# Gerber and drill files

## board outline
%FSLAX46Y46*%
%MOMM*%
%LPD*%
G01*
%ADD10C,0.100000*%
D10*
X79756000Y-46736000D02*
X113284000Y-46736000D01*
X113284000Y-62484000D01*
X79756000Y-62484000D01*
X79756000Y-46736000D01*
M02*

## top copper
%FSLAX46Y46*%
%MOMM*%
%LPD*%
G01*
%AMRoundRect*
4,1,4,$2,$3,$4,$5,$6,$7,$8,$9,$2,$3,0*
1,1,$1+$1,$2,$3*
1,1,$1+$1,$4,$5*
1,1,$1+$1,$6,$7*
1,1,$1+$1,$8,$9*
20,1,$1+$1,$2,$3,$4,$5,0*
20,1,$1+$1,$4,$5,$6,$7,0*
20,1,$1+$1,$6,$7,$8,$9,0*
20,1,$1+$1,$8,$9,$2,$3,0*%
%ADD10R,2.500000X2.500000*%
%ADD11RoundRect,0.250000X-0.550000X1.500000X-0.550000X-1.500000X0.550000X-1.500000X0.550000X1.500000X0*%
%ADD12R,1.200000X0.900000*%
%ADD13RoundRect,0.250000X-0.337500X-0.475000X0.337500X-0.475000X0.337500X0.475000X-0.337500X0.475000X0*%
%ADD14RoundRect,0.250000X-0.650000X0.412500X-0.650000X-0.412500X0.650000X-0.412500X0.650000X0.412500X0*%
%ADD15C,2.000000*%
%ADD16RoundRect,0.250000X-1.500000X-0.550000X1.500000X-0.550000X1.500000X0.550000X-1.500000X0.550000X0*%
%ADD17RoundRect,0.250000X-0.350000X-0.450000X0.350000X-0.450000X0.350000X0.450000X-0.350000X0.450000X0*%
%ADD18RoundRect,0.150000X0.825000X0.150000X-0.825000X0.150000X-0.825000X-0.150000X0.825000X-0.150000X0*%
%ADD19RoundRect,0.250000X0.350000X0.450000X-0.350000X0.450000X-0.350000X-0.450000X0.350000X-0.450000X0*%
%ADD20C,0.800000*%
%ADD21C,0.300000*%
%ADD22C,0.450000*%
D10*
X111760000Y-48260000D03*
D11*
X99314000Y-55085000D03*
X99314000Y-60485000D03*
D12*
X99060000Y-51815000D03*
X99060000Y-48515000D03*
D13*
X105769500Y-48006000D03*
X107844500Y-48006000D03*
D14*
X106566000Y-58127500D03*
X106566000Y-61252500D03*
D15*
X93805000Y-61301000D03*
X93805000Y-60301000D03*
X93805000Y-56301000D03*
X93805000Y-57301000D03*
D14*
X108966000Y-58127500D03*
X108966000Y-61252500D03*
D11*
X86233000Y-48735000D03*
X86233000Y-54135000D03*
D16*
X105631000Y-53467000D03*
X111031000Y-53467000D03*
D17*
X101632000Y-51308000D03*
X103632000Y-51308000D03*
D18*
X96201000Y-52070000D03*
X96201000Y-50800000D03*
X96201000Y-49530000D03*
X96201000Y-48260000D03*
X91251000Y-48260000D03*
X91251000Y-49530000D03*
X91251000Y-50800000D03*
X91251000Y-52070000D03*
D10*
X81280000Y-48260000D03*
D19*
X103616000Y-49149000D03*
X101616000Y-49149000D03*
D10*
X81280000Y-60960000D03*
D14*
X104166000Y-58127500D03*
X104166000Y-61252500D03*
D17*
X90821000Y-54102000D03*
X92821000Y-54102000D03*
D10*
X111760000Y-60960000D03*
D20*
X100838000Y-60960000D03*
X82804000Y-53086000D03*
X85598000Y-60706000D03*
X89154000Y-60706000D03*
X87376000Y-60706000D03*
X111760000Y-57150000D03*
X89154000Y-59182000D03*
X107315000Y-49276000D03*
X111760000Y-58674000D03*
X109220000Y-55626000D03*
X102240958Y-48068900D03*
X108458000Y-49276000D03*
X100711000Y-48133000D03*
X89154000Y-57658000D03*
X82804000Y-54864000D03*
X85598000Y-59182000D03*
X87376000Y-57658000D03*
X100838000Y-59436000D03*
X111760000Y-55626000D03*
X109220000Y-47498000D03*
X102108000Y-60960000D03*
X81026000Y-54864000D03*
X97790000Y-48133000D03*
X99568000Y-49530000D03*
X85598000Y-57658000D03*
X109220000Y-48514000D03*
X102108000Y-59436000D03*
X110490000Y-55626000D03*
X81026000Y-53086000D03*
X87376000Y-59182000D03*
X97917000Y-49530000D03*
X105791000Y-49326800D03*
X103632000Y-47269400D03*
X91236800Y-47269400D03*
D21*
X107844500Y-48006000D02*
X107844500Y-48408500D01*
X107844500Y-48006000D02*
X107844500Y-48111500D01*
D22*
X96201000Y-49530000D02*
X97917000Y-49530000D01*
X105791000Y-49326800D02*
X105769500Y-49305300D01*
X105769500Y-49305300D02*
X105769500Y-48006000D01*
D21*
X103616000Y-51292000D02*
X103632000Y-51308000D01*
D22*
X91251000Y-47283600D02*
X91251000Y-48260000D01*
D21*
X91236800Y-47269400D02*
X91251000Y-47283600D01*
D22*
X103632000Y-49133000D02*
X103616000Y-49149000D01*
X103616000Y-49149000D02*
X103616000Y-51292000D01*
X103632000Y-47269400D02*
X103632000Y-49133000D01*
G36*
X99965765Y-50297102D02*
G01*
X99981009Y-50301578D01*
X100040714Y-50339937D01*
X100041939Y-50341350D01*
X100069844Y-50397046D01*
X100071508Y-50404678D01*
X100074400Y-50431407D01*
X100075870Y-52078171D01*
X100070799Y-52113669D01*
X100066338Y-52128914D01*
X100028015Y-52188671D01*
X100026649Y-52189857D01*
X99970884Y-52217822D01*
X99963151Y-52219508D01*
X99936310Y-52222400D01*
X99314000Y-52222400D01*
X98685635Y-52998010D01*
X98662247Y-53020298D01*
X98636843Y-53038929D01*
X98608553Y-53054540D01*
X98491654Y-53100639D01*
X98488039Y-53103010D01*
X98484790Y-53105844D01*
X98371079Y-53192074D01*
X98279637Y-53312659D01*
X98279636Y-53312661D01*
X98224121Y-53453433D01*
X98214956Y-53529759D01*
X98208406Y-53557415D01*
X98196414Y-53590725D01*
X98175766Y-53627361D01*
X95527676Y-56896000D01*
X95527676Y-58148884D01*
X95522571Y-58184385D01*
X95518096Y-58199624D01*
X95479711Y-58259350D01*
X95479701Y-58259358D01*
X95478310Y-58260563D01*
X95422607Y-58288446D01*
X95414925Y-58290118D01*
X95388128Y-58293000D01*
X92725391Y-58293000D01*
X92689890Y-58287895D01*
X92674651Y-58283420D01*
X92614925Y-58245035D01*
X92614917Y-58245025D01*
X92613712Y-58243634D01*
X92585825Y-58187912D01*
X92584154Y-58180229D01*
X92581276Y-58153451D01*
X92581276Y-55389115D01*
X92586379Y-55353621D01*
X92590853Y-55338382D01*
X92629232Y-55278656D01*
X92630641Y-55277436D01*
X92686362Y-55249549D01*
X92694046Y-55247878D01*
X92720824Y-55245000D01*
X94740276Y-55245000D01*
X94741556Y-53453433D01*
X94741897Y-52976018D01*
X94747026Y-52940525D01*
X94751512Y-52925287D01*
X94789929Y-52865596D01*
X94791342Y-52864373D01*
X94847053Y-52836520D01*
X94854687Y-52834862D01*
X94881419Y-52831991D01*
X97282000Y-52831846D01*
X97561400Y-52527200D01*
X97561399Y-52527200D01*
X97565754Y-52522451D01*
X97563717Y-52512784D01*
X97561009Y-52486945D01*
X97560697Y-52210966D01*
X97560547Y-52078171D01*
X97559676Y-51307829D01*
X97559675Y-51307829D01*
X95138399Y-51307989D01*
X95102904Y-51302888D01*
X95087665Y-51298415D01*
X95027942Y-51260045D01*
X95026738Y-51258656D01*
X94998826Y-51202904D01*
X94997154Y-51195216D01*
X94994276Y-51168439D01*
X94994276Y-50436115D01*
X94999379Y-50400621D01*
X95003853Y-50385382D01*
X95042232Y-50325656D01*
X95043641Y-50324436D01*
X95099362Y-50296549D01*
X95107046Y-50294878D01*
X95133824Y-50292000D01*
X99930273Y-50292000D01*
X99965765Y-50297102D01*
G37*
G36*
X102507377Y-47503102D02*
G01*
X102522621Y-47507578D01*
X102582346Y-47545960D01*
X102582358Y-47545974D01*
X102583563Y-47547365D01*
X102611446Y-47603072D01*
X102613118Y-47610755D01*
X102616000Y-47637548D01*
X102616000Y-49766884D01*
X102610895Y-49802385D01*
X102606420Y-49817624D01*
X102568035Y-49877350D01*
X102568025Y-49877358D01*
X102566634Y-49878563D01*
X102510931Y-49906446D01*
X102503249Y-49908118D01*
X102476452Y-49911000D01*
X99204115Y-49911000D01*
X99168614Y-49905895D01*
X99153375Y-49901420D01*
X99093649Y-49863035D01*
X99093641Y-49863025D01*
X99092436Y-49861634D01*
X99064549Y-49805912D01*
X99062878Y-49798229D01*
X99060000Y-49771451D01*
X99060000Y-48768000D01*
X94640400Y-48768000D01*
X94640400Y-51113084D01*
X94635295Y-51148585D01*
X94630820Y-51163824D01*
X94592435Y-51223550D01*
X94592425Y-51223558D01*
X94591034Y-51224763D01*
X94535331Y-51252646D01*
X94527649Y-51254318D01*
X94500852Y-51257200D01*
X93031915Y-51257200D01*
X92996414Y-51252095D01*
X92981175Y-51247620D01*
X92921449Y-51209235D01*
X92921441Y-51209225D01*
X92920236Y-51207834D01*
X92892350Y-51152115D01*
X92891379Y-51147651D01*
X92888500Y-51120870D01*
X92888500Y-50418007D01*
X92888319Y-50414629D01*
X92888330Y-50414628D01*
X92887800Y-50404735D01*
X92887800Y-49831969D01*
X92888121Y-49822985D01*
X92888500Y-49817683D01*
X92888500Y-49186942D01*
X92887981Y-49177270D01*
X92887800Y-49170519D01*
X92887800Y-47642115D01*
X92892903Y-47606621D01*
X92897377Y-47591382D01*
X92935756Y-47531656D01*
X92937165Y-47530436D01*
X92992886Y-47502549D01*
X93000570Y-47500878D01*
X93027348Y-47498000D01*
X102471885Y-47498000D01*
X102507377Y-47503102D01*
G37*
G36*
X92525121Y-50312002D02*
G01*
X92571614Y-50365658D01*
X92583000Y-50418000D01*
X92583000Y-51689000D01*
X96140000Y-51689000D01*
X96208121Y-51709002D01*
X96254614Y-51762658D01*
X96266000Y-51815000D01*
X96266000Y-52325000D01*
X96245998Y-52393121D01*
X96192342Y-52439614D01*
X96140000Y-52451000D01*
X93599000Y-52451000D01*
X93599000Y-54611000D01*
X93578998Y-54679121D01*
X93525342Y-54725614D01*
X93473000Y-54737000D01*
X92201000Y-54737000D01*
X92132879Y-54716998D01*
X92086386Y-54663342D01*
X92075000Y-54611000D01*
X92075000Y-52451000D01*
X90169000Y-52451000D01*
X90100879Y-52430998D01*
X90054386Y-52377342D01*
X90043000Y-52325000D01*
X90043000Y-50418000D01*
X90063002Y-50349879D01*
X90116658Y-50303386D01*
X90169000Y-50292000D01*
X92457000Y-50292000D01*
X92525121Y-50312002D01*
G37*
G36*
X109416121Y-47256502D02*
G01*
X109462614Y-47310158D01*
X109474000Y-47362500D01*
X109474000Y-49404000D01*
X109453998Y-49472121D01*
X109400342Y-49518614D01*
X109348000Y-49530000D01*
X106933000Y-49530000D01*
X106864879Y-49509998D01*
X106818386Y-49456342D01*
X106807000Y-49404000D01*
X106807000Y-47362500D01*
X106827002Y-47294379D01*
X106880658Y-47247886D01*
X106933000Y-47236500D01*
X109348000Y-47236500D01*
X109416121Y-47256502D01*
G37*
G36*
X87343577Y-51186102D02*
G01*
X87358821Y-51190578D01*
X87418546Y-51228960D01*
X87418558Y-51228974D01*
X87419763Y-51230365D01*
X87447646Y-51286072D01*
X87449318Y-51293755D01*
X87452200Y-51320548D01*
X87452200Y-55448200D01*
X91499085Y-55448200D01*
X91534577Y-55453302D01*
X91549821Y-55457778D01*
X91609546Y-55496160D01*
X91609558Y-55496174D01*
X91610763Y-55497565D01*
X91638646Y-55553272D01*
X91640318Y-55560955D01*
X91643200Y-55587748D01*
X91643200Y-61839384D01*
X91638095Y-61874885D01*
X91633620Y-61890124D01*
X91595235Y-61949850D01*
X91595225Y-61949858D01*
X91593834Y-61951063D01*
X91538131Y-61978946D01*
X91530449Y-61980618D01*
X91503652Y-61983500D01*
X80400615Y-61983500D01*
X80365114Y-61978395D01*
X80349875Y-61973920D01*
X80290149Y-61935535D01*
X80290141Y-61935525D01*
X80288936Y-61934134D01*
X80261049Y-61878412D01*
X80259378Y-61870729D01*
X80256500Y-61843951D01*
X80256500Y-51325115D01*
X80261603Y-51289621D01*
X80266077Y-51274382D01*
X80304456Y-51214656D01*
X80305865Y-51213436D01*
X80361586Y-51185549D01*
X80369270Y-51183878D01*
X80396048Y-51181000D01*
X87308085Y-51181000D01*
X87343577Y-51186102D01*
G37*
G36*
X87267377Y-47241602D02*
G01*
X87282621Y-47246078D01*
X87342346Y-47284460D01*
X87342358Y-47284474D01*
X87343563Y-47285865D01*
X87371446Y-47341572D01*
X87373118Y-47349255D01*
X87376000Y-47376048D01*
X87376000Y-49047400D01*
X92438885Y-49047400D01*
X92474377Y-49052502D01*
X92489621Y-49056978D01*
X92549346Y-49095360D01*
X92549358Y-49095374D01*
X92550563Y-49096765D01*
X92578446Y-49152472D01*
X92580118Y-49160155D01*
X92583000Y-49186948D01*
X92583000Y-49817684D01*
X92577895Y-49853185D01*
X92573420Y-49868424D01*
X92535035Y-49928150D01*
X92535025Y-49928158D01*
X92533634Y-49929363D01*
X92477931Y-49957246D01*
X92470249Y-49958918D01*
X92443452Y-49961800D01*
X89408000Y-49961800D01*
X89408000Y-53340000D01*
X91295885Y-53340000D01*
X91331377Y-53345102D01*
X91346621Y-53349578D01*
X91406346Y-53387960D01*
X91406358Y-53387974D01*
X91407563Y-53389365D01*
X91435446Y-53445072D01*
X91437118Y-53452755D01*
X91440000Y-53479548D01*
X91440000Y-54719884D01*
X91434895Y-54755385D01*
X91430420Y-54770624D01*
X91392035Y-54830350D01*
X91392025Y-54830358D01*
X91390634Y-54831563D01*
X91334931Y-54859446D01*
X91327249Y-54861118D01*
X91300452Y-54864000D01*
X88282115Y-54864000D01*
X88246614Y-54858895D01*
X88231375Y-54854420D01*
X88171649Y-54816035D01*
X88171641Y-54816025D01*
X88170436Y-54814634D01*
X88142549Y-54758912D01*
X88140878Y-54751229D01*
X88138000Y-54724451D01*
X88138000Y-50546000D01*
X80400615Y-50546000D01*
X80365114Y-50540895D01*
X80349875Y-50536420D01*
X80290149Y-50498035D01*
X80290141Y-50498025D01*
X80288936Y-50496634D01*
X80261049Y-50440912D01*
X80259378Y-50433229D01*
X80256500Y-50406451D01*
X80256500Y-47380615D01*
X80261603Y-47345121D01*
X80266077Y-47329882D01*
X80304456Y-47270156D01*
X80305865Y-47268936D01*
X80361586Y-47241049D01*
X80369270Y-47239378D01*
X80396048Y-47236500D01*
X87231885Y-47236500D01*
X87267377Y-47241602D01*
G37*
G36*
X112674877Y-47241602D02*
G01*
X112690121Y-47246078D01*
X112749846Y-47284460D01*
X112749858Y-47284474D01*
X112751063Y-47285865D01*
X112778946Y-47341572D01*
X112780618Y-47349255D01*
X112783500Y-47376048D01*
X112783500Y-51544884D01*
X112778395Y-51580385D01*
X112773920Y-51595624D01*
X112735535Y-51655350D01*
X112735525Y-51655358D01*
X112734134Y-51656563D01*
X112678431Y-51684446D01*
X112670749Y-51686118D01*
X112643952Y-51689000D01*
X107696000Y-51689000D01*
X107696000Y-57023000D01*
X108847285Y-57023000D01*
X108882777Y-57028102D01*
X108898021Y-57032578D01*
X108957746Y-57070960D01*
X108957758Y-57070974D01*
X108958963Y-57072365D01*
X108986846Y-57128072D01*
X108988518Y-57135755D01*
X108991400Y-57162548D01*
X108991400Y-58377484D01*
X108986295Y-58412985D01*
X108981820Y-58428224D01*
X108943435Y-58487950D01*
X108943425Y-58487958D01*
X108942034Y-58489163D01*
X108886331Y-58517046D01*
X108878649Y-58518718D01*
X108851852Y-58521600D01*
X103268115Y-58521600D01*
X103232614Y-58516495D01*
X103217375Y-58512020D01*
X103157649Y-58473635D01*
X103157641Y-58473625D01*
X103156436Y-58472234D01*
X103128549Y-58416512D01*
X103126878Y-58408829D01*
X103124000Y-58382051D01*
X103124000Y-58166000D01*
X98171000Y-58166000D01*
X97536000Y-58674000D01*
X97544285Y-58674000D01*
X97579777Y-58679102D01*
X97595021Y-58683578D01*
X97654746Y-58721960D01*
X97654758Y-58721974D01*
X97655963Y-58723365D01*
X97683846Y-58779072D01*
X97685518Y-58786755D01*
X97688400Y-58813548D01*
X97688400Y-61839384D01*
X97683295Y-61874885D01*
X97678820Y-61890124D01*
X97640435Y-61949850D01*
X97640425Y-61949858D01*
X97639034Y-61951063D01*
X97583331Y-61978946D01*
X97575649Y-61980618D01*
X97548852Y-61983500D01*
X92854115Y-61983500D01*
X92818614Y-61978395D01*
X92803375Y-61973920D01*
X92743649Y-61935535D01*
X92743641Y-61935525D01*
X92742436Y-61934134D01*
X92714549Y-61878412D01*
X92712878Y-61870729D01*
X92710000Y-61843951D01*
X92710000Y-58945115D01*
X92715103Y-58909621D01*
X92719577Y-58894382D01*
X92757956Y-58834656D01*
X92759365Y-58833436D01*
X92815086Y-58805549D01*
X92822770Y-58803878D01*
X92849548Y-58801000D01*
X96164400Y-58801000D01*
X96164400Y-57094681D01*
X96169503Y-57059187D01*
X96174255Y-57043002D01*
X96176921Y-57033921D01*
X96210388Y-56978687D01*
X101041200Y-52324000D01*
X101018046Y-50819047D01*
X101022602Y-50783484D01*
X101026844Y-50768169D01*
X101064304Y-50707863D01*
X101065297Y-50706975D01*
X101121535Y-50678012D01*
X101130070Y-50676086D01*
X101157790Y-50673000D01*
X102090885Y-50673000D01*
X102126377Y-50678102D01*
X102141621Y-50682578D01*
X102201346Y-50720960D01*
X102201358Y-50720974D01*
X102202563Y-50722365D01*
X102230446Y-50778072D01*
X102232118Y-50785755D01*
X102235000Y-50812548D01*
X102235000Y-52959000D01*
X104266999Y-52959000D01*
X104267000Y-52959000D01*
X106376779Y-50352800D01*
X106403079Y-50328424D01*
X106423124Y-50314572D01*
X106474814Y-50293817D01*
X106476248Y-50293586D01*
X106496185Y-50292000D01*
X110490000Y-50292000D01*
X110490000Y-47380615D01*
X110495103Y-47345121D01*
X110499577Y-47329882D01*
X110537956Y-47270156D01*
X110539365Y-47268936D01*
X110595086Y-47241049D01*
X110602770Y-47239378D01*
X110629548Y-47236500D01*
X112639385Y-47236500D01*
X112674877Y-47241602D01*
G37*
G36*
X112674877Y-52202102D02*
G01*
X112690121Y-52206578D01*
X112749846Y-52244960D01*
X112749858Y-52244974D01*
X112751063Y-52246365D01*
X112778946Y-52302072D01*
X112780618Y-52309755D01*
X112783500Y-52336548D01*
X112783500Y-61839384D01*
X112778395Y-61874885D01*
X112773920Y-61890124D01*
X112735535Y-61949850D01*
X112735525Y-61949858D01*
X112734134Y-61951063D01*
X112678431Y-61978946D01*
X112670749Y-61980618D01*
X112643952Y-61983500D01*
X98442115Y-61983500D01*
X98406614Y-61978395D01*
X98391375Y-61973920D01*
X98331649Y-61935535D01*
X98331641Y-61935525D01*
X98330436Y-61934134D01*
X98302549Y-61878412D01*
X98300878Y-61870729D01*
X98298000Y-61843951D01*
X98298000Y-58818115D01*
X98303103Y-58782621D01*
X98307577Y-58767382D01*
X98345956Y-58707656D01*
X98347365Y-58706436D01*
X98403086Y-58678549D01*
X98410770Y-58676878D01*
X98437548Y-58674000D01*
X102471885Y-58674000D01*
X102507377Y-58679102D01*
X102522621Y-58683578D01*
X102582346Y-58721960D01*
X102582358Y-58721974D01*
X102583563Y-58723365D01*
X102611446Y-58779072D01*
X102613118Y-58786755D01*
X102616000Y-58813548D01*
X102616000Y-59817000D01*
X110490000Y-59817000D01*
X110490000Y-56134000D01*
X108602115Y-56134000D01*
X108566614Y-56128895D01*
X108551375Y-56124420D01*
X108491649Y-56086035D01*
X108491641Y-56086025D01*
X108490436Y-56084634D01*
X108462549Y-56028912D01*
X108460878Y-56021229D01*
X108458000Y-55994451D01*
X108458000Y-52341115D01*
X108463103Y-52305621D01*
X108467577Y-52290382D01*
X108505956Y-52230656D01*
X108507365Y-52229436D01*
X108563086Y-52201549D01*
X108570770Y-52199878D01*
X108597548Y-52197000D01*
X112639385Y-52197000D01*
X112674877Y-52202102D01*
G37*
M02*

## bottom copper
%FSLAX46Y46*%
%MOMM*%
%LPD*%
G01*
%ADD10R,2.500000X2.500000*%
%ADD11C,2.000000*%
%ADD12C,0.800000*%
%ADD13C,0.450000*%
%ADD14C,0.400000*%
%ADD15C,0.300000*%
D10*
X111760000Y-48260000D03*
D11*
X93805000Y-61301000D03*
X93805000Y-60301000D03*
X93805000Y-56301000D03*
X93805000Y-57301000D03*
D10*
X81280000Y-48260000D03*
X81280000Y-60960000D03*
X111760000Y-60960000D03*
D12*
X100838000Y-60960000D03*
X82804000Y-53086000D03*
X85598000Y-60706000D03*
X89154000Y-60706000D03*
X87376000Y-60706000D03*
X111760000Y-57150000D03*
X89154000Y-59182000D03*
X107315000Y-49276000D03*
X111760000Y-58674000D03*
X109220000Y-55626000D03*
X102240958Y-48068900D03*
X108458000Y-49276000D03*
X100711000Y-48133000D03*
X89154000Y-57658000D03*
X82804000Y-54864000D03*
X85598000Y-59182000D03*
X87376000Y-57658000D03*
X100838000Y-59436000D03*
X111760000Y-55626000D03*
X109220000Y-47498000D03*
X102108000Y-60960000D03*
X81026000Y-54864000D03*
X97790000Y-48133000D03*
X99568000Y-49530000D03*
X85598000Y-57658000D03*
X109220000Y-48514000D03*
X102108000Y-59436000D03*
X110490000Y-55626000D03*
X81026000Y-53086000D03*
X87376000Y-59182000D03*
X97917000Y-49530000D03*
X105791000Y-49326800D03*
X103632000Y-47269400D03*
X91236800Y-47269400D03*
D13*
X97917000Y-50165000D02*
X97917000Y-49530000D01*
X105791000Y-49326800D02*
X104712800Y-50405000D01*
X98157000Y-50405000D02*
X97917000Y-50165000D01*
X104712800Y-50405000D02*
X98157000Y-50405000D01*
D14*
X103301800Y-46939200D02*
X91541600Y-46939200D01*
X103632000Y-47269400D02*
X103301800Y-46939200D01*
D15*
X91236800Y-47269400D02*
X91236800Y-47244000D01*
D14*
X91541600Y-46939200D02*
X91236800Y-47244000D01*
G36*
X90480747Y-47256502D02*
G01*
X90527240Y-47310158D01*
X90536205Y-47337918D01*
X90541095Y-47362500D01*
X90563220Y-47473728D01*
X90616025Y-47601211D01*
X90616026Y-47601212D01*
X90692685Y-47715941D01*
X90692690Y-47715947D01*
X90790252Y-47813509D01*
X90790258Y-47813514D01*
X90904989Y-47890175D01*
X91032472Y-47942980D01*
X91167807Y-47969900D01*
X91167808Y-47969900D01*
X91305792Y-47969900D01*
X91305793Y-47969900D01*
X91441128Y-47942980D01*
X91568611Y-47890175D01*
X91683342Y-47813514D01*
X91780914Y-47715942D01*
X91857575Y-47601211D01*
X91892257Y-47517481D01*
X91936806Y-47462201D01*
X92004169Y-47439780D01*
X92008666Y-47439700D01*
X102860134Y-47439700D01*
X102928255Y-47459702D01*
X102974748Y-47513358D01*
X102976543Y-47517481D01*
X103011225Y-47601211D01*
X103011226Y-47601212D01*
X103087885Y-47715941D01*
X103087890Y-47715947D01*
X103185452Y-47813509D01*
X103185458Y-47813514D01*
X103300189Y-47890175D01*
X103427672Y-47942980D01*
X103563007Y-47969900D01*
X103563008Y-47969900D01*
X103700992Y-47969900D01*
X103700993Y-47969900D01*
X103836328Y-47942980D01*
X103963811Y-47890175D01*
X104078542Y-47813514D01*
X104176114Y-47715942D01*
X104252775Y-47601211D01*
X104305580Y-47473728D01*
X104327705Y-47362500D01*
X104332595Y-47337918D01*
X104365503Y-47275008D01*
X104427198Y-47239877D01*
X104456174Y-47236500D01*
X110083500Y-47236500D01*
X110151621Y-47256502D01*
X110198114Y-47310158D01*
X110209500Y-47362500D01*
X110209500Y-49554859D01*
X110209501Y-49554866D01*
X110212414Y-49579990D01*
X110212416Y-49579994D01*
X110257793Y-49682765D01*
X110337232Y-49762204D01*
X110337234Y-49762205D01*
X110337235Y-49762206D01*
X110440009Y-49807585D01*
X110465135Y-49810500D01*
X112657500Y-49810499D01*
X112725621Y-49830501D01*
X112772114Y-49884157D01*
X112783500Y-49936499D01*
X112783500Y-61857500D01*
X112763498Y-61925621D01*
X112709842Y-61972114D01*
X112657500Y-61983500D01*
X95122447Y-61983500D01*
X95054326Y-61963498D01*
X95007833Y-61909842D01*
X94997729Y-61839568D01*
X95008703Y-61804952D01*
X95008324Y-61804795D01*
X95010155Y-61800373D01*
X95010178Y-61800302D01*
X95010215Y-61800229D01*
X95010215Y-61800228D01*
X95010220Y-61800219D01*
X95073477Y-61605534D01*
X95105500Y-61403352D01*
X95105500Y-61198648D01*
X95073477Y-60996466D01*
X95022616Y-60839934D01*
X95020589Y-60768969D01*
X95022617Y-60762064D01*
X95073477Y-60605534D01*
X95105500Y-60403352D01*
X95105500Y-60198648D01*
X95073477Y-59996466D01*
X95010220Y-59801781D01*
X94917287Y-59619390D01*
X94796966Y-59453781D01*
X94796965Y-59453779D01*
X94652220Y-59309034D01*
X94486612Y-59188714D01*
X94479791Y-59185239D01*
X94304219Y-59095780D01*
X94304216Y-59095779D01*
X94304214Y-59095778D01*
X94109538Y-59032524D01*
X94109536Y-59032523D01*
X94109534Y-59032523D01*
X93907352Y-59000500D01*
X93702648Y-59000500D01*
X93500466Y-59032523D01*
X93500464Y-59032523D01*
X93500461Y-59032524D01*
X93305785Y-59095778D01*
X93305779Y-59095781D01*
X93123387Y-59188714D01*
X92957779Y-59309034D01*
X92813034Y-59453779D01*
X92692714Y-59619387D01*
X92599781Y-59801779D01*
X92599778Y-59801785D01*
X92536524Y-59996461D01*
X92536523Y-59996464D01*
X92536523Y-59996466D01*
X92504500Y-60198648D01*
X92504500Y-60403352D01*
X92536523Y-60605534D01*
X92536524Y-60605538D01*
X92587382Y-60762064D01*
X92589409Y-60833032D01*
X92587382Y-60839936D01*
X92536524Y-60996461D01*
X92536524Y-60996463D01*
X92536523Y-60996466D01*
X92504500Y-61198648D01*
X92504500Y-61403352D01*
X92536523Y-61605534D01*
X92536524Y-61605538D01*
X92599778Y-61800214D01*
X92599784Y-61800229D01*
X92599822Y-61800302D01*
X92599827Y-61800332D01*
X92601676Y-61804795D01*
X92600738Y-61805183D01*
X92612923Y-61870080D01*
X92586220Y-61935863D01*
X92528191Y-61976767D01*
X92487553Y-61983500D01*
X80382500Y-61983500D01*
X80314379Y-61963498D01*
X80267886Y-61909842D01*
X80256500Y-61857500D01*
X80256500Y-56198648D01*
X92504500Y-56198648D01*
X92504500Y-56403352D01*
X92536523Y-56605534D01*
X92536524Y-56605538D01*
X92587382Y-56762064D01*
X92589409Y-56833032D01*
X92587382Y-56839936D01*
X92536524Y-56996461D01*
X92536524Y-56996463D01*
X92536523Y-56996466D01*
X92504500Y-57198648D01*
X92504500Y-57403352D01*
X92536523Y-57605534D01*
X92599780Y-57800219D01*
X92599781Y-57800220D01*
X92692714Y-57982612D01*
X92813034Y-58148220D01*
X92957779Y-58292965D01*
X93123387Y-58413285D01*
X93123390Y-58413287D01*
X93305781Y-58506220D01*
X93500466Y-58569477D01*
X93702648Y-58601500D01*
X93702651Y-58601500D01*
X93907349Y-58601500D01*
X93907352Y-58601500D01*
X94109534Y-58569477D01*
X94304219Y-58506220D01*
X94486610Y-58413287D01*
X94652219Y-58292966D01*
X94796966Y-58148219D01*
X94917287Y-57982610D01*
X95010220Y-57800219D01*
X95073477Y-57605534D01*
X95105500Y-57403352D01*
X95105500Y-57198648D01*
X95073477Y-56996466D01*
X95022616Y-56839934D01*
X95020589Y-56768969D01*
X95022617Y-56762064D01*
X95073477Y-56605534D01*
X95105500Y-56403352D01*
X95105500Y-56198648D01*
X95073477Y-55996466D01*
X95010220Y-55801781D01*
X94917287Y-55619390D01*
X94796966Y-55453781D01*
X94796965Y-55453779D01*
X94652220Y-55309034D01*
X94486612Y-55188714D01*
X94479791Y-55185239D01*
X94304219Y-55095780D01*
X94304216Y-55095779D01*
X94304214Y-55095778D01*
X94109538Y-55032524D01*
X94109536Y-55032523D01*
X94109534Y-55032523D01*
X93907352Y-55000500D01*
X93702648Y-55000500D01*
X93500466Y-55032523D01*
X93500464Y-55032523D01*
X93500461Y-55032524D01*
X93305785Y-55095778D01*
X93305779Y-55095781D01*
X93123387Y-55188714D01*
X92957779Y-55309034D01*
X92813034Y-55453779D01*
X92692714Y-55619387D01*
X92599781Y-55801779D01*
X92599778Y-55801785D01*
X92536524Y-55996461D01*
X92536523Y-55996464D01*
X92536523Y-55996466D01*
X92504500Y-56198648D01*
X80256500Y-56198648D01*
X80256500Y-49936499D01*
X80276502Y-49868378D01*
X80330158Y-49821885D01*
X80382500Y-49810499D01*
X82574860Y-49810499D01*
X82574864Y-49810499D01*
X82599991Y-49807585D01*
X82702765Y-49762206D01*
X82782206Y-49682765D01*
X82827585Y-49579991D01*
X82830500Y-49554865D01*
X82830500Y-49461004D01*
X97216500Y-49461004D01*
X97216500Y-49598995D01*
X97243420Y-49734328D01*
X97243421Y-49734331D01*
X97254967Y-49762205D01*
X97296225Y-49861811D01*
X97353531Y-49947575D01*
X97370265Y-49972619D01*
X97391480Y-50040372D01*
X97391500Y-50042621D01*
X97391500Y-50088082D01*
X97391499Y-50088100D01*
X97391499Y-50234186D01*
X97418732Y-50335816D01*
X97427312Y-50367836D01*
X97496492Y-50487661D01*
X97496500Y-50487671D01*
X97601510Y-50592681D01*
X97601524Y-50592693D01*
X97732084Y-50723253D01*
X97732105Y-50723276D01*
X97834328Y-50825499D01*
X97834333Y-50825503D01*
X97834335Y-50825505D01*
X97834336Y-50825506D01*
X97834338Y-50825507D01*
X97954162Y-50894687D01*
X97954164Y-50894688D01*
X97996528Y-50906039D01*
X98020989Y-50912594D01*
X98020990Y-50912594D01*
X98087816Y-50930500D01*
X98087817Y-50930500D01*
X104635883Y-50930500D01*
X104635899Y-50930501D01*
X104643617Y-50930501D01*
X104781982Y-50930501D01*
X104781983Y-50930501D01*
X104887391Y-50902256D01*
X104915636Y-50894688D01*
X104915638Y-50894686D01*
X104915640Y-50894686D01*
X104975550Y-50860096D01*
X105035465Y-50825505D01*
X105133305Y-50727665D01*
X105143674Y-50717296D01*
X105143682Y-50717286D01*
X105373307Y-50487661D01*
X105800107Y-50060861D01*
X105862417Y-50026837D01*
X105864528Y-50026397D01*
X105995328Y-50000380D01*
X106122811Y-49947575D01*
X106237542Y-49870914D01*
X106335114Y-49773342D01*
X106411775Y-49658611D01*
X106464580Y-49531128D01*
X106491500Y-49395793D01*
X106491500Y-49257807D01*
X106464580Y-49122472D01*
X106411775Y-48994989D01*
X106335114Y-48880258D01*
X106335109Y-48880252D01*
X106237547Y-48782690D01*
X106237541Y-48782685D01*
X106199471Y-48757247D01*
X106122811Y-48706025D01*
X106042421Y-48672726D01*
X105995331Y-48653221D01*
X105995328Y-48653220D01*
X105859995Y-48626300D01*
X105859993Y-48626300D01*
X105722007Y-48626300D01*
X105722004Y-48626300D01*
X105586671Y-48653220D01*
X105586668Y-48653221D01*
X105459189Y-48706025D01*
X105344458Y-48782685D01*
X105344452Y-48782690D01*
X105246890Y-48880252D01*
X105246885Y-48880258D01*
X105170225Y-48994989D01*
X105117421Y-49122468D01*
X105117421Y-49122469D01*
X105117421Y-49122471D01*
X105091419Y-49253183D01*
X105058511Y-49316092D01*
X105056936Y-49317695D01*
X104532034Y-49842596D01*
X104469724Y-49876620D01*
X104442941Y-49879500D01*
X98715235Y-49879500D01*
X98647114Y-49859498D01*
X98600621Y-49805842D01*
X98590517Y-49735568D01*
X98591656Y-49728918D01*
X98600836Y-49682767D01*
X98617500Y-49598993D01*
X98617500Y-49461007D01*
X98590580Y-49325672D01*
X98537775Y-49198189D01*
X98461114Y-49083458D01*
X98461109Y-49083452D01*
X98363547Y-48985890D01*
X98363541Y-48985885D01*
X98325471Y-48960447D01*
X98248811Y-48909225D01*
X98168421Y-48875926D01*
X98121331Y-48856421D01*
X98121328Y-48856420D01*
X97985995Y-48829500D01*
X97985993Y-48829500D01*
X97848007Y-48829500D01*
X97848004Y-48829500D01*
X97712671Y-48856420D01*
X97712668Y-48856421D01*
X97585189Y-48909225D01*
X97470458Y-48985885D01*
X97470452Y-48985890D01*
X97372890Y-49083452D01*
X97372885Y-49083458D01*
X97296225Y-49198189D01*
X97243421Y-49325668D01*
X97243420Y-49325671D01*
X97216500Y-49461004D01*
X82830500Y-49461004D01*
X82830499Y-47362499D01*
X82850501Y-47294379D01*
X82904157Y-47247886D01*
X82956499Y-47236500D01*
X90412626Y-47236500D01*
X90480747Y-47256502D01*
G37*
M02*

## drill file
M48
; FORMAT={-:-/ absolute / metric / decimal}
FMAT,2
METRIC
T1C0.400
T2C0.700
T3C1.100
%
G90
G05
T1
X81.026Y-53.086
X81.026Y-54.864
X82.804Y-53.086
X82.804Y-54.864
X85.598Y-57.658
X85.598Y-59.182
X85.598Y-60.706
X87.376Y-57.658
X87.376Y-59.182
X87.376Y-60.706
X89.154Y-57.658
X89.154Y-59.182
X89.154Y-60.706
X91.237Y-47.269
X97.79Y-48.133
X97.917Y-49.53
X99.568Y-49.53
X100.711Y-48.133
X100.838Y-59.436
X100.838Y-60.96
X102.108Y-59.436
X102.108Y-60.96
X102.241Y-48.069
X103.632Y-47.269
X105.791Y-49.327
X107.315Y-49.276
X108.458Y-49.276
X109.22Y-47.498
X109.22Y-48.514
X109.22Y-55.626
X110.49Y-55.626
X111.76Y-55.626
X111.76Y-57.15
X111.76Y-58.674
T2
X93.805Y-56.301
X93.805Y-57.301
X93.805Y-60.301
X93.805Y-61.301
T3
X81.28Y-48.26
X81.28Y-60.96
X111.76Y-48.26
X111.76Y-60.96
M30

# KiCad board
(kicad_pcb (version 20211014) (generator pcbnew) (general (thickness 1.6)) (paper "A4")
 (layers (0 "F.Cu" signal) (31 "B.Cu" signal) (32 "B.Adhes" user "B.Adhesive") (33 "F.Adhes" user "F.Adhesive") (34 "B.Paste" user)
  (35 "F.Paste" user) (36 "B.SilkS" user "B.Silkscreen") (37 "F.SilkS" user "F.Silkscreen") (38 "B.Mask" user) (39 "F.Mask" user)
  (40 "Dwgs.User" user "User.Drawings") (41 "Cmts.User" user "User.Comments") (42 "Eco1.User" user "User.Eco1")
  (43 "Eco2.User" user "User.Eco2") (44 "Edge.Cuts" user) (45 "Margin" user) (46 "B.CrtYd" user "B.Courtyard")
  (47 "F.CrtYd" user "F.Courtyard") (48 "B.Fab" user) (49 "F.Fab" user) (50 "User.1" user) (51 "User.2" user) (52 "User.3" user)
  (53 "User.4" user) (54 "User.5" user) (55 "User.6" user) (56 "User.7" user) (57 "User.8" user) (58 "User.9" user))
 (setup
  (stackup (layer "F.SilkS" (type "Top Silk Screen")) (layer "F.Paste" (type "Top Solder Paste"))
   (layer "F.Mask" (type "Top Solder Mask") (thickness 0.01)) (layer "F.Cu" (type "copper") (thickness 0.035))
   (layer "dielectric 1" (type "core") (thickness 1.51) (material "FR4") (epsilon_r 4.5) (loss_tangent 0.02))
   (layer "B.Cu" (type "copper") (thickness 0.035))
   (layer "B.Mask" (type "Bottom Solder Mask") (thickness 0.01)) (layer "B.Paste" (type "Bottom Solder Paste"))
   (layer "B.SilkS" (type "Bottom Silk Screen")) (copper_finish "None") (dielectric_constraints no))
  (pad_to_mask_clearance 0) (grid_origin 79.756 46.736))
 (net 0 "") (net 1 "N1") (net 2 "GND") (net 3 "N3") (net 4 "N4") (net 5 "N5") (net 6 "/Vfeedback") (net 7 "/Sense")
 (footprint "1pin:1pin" (layer "F.Cu") (at 111.76 48.26)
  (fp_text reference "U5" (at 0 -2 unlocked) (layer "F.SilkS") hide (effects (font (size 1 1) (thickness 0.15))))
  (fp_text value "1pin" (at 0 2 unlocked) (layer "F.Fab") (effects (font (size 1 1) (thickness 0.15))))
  (pad "1" thru_hole rect (at 0 0) (size 2.5 2.5) (drill 1.1) (layers *.Cu *.Mask) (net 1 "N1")))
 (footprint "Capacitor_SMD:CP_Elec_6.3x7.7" (layer "F.Cu") (at 99.314 57.785 -90)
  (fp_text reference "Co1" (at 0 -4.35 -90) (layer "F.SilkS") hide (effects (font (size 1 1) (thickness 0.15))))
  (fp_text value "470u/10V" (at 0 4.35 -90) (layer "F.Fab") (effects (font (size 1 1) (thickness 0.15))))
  (pad "1" smd roundrect (at -2.7 0 270) (size 3.5 1.6) (layers "F.Cu" "F.Paste" "F.Mask") (roundrect_rratio 0.15625) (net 1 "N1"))
  (pad "2" smd roundrect (at 2.7 0 270) (size 3.5 1.6) (layers "F.Cu" "F.Paste" "F.Mask") (roundrect_rratio 0.15625) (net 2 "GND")))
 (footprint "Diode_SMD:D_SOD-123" (layer "F.Cu") (at 99.06 50.165 90)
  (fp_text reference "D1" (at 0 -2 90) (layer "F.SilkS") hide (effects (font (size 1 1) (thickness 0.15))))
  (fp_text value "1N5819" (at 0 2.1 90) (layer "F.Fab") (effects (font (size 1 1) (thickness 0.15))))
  (pad "1" smd rect (at -1.65 0 90) (size 0.9 1.2) (layers "F.Cu" "F.Paste" "F.Mask") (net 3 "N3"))
  (pad "2" smd rect (at 1.65 0 90) (size 0.9 1.2) (layers "F.Cu" "F.Paste" "F.Mask") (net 2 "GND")))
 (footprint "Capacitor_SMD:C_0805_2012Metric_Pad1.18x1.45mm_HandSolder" (layer "F.Cu") (at 106.807 48.006)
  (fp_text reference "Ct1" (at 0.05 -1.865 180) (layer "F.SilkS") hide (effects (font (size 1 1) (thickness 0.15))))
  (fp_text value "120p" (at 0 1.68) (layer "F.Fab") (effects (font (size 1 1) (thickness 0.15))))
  (pad "1" smd roundrect (at -1.0375 0) (size 1.175 1.45) (layers "F.Cu" "F.Paste" "F.Mask") (roundrect_rratio 0.2127659574) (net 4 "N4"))
  (pad "2" smd roundrect (at 1.0375 0) (size 1.175 1.45) (layers "F.Cu" "F.Paste" "F.Mask") (roundrect_rratio 0.2127659574) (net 2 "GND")))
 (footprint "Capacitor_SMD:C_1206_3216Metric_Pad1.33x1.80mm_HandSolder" (layer "F.Cu") (at 106.566 59.69 -90)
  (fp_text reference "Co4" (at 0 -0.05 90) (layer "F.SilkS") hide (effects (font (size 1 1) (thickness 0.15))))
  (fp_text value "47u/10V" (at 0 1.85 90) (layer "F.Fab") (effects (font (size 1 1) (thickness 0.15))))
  (pad "1" smd roundrect (at -1.5625 0 270) (size 1.325 1.8) (layers "F.Cu" "F.Paste" "F.Mask") (roundrect_rratio 0.188679) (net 1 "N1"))
  (pad "2" smd roundrect (at 1.5625 0 270) (size 1.325 1.8) (layers "F.Cu" "F.Paste" "F.Mask") (roundrect_rratio 0.188679) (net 2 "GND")))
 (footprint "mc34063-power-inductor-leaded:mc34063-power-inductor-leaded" (layer "F.Cu") (at 93.805 58.801)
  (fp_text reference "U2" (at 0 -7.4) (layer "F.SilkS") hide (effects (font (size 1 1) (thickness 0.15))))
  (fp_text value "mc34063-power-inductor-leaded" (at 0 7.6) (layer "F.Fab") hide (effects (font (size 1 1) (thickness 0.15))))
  (pad "1" thru_hole circle (at 0 2.5 180) (size 2 2) (drill 0.7) (layers *.Cu *.Mask) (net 1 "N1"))
  (pad "1" thru_hole circle (at 0 1.5 180) (size 2 2) (drill 0.7) (layers *.Cu *.Mask) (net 1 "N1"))
  (pad "2" thru_hole circle (at 0 -2.5 180) (size 2 2) (drill 0.7) (layers *.Cu *.Mask) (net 3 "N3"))
  (pad "2" thru_hole circle (at 0 -1.5 180) (size 2 2) (drill 0.7) (layers *.Cu *.Mask) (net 3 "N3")))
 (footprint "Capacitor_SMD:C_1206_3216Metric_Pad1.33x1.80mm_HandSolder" (layer "F.Cu") (at 108.966 59.69 -90)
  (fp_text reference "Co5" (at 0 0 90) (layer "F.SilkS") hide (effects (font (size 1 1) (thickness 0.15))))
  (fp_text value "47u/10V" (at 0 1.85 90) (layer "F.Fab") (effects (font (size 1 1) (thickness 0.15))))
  (pad "1" smd roundrect (at -1.5625 0 270) (size 1.325 1.8) (layers "F.Cu" "F.Paste" "F.Mask") (roundrect_rratio 0.188679) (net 1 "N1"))
  (pad "2" smd roundrect (at 1.5625 0 270) (size 1.325 1.8) (layers "F.Cu" "F.Paste" "F.Mask") (roundrect_rratio 0.188679) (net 2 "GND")))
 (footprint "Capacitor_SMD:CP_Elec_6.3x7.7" (layer "F.Cu") (at 86.233 51.435 -90)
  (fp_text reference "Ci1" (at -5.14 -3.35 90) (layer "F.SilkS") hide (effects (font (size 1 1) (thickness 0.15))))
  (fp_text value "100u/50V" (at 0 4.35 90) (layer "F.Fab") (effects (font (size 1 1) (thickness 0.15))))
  (pad "1" smd roundrect (at -2.7 0 270) (size 3.5 1.6) (layers "F.Cu" "F.Paste" "F.Mask") (roundrect_rratio 0.15625) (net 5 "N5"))
  (pad "2" smd roundrect (at 2.7 0 270) (size 3.5 1.6) (layers "F.Cu" "F.Paste" "F.Mask") (roundrect_rratio 0.15625) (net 2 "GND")))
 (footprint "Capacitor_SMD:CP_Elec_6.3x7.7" (layer "F.Cu") (at 108.331 53.467)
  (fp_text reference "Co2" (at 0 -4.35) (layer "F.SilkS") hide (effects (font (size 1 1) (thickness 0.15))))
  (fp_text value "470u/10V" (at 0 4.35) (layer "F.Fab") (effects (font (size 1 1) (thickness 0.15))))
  (pad "1" smd roundrect (at -2.7 0) (size 3.5 1.6) (layers "F.Cu" "F.Paste" "F.Mask") (roundrect_rratio 0.15625) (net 1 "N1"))
  (pad "2" smd roundrect (at 2.7 0) (size 3.5 1.6) (layers "F.Cu" "F.Paste" "F.Mask") (roundrect_rratio 0.15625) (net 2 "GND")))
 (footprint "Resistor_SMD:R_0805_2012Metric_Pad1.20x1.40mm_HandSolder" (layer "F.Cu") (at 102.632 51.308)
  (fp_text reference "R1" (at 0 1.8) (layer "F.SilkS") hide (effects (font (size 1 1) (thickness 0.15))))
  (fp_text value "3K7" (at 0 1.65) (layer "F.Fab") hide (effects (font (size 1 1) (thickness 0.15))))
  (pad "1" smd roundrect (at -1 0) (size 1.2 1.4) (layers "F.Cu" "F.Paste" "F.Mask") (roundrect_rratio 0.2083333333) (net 1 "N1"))
  (pad "2" smd roundrect (at 1 0) (size 1.2 1.4) (layers "F.Cu" "F.Paste" "F.Mask") (roundrect_rratio 0.2083333333) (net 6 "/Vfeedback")))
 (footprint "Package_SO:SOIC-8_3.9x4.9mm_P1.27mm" (layer "F.Cu") (at 93.726 50.165 180)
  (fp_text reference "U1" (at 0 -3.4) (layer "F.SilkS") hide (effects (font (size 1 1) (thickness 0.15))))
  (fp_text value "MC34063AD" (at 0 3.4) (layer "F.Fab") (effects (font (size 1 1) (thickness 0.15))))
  (pad "1" smd roundrect (at -2.475 -1.905 180) (size 1.95 0.6) (layers "F.Cu" "F.Paste" "F.Mask") (roundrect_rratio 0.25) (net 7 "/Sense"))
  (pad "2" smd roundrect (at -2.475 -0.635 180) (size 1.95 0.6) (layers "F.Cu" "F.Paste" "F.Mask") (roundrect_rratio 0.25) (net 3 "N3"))
  (pad "3" smd roundrect (at -2.475 0.635 180) (size 1.95 0.6) (layers "F.Cu" "F.Paste" "F.Mask") (roundrect_rratio 0.25) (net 4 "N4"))
  (pad "4" smd roundrect (at -2.475 1.905 180) (size 1.95 0.6) (layers "F.Cu" "F.Paste" "F.Mask") (roundrect_rratio 0.25) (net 2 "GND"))
  (pad "5" smd roundrect (at 2.475 1.905 180) (size 1.95 0.6) (layers "F.Cu" "F.Paste" "F.Mask") (roundrect_rratio 0.25)
   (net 6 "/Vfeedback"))
  (pad "6" smd roundrect (at 2.475 0.635 180) (size 1.95 0.6) (layers "F.Cu" "F.Paste" "F.Mask") (roundrect_rratio 0.25) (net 5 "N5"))
  (pad "7" smd roundrect (at 2.475 -0.635 180) (size 1.95 0.6) (layers "F.Cu" "F.Paste" "F.Mask") (roundrect_rratio 0.25) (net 7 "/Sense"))
  (pad "8" smd roundrect (at 2.475 -1.905 180) (size 1.95 0.6) (layers "F.Cu" "F.Paste" "F.Mask") (roundrect_rratio 0.25) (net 7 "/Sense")))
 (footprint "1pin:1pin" (layer "F.Cu") (at 81.28 48.26)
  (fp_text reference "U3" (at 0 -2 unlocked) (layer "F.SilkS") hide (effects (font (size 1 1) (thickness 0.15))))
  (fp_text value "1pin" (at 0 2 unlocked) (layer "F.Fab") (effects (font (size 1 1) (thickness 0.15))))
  (pad "1" thru_hole rect (at 0 0) (size 2.5 2.5) (drill 1.1) (layers *.Cu *.Mask) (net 5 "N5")))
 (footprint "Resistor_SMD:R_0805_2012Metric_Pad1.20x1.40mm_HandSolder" (layer "F.Cu") (at 102.616 49.149 180)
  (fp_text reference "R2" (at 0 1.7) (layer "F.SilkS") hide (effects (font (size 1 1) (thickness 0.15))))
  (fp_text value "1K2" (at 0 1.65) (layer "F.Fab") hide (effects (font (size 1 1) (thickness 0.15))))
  (pad "1" smd roundrect (at -1 0 180) (size 1.2 1.4) (layers "F.Cu" "F.Paste" "F.Mask") (roundrect_rratio 0.2083333333)
   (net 6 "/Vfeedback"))
  (pad "2" smd roundrect (at 1 0 180) (size 1.2 1.4) (layers "F.Cu" "F.Paste" "F.Mask") (roundrect_rratio 0.2083333333) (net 2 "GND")))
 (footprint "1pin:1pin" (layer "F.Cu") (at 81.28 60.96)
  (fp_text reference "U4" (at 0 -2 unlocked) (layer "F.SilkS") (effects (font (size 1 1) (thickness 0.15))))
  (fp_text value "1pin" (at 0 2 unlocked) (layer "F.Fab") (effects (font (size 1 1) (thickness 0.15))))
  (pad "1" thru_hole rect (at 0 0) (size 2.5 2.5) (drill 1.1) (layers *.Cu *.Mask) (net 2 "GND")))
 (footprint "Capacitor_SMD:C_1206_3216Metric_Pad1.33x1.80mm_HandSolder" (layer "F.Cu") (at 104.166 59.69 -90)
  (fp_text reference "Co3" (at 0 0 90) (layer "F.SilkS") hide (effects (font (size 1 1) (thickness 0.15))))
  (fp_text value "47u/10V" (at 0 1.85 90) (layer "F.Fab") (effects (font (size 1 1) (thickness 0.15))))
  (pad "1" smd roundrect (at -1.5625 0 270) (size 1.325 1.8) (layers "F.Cu" "F.Paste" "F.Mask") (roundrect_rratio 0.188679) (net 1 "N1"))
  (pad "2" smd roundrect (at 1.5625 0 270) (size 1.325 1.8) (layers "F.Cu" "F.Paste" "F.Mask") (roundrect_rratio 0.188679) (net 2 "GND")))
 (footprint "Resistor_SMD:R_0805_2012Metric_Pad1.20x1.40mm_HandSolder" (layer "F.Cu") (at 91.821 54.102)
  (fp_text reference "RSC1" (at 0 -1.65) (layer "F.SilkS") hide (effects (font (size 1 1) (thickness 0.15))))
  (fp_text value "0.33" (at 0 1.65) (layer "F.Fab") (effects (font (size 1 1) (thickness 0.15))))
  (pad "1" smd roundrect (at -1 0) (size 1.2 1.4) (layers "F.Cu" "F.Paste" "F.Mask") (roundrect_rratio 0.2083333333) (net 5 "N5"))
  (pad "2" smd roundrect (at 1 0) (size 1.2 1.4) (layers "F.Cu" "F.Paste" "F.Mask") (roundrect_rratio 0.2083333333) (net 7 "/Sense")))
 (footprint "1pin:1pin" (layer "F.Cu") (at 111.76 60.96)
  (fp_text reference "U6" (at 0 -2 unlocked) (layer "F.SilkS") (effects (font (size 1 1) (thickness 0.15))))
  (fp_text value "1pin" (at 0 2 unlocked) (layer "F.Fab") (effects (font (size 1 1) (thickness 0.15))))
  (pad "1" thru_hole rect (at 0 0) (size 2.5 2.5) (drill 1.1) (layers *.Cu *.Mask) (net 2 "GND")))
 (gr_rect (start 79.756 46.736) (end 113.284 62.484) (layer "Edge.Cuts") (width 0.1) (fill none))
 (segment (start 107.8445 48.006) (end 107.8445 48.4085) (width 0.3) (layer "F.Cu") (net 2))
 (segment (start 107.8445 48.006) (end 107.8445 48.1115) (width 0.3) (layer "F.Cu") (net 2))
 (via (at 100.838 60.96) (size 0.8) (drill 0.4) (layers "F.Cu" "B.Cu") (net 2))
 (via (at 82.804 53.086) (size 0.8) (drill 0.4) (layers "F.Cu" "B.Cu") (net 2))
 (via (at 85.598 60.706) (size 0.8) (drill 0.4) (layers "F.Cu" "B.Cu") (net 2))
 (via (at 89.154 60.706) (size 0.8) (drill 0.4) (layers "F.Cu" "B.Cu") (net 2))
 (via (at 87.376 60.706) (size 0.8) (drill 0.4) (layers "F.Cu" "B.Cu") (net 2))
 (via (at 111.76 57.15) (size 0.8) (drill 0.4) (layers "F.Cu" "B.Cu") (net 2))
 (via (at 89.154 59.182) (size 0.8) (drill 0.4) (layers "F.Cu" "B.Cu") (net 2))
 (via (at 107.315 49.276) (size 0.8) (drill 0.4) (layers "F.Cu" "B.Cu") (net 2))
 (via (at 111.76 58.674) (size 0.8) (drill 0.4) (layers "F.Cu" "B.Cu") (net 2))
 (via (at 109.22 55.626) (size 0.8) (drill 0.4) (layers "F.Cu" "B.Cu") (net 2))
 (via (at 102.240958 48.0689) (size 0.8) (drill 0.4) (layers "F.Cu" "B.Cu") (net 2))
 (via (at 108.458 49.276) (size 0.8) (drill 0.4) (layers "F.Cu" "B.Cu") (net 2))
 (via (at 100.711 48.133) (size 0.8) (drill 0.4) (layers "F.Cu" "B.Cu") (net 2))
 (via (at 89.154 57.658) (size 0.8) (drill 0.4) (layers "F.Cu" "B.Cu") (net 2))
 (via (at 82.804 54.864) (size 0.8) (drill 0.4) (layers "F.Cu" "B.Cu") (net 2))
 (via (at 85.598 59.182) (size 0.8) (drill 0.4) (layers "F.Cu" "B.Cu") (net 2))
 (via (at 87.376 57.658) (size 0.8) (drill 0.4) (layers "F.Cu" "B.Cu") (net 2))
 (via (at 100.838 59.436) (size 0.8) (drill 0.4) (layers "F.Cu" "B.Cu") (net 2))
 (via (at 111.76 55.626) (size 0.8) (drill 0.4) (layers "F.Cu" "B.Cu") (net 2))
 (via (at 109.22 47.498) (size 0.8) (drill 0.4) (layers "F.Cu" "B.Cu") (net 2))
 (via (at 102.108 60.96) (size 0.8) (drill 0.4) (layers "F.Cu" "B.Cu") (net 2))
 (via (at 81.026 54.864) (size 0.8) (drill 0.4) (layers "F.Cu" "B.Cu") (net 2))
 (via (at 97.79 48.133) (size 0.8) (drill 0.4) (layers "F.Cu" "B.Cu") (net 2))
 (via (at 99.568 49.53) (size 0.8) (drill 0.4) (layers "F.Cu" "B.Cu") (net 2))
 (via (at 85.598 57.658) (size 0.8) (drill 0.4) (layers "F.Cu" "B.Cu") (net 2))
 (via (at 109.22 48.514) (size 0.8) (drill 0.4) (layers "F.Cu" "B.Cu") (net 2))
 (via (at 102.108 59.436) (size 0.8) (drill 0.4) (layers "F.Cu" "B.Cu") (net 2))
 (via (at 110.49 55.626) (size 0.8) (drill 0.4) (layers "F.Cu" "B.Cu") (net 2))
 (via (at 81.026 53.086) (size 0.8) (drill 0.4) (layers "F.Cu" "B.Cu") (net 2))
 (via (at 87.376 59.182) (size 0.8) (drill 0.4) (layers "F.Cu" "B.Cu") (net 2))
 (segment (start 96.201 49.53) (end 97.917 49.53) (width 0.45) (layer "F.Cu") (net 4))
 (segment (start 105.791 49.3268) (end 105.7695 49.3053) (width 0.45) (layer "F.Cu") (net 4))
 (segment (start 105.7695 49.3053) (end 105.7695 48.006) (width 0.45) (layer "F.Cu") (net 4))
 (via (at 97.917 49.53) (size 0.8) (drill 0.4) (layers "F.Cu" "B.Cu") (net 4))
 (via (at 105.791 49.3268) (size 0.8) (drill 0.4) (layers "F.Cu" "B.Cu") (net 4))
 (segment (start 97.917 50.165) (end 97.917 49.53) (width 0.45) (layer "B.Cu") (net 4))
 (segment (start 105.791 49.3268) (end 104.7128 50.405) (width 0.45) (layer "B.Cu") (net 4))
 (segment (start 98.157 50.405) (end 97.917 50.165) (width 0.45) (layer "B.Cu") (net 4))
 (segment (start 104.7128 50.405) (end 98.157 50.405) (width 0.45) (layer "B.Cu") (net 4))
 (segment (start 103.616 51.292) (end 103.632 51.308) (width 0.3) (layer "F.Cu") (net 6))
 (segment (start 91.251 47.2836) (end 91.251 48.26) (width 0.45) (layer "F.Cu") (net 6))
 (segment (start 91.2368 47.2694) (end 91.251 47.2836) (width 0.3) (layer "F.Cu") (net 6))
 (segment (start 103.632 49.133) (end 103.616 49.149) (width 0.45) (layer "F.Cu") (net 6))
 (segment (start 103.616 49.149) (end 103.616 51.292) (width 0.45) (layer "F.Cu") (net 6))
 (segment (start 103.632 47.2694) (end 103.632 49.133) (width 0.45) (layer "F.Cu") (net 6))
 (via (at 103.632 47.2694) (size 0.8) (drill 0.4) (layers "F.Cu" "B.Cu") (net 6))
 (via (at 91.2368 47.2694) (size 0.8) (drill 0.4) (layers "F.Cu" "B.Cu") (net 6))
 (segment (start 103.3018 46.9392) (end 91.5416 46.9392) (width 0.4) (layer "B.Cu") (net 6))
 (segment (start 103.632 47.2694) (end 103.3018 46.9392) (width 0.4) (layer "B.Cu") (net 6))
 (segment (start 91.2368 47.2694) (end 91.2368 47.244) (width 0.3) (layer "B.Cu") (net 6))
 (segment (start 91.5416 46.9392) (end 91.2368 47.244) (width 0.4) (layer "B.Cu") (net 6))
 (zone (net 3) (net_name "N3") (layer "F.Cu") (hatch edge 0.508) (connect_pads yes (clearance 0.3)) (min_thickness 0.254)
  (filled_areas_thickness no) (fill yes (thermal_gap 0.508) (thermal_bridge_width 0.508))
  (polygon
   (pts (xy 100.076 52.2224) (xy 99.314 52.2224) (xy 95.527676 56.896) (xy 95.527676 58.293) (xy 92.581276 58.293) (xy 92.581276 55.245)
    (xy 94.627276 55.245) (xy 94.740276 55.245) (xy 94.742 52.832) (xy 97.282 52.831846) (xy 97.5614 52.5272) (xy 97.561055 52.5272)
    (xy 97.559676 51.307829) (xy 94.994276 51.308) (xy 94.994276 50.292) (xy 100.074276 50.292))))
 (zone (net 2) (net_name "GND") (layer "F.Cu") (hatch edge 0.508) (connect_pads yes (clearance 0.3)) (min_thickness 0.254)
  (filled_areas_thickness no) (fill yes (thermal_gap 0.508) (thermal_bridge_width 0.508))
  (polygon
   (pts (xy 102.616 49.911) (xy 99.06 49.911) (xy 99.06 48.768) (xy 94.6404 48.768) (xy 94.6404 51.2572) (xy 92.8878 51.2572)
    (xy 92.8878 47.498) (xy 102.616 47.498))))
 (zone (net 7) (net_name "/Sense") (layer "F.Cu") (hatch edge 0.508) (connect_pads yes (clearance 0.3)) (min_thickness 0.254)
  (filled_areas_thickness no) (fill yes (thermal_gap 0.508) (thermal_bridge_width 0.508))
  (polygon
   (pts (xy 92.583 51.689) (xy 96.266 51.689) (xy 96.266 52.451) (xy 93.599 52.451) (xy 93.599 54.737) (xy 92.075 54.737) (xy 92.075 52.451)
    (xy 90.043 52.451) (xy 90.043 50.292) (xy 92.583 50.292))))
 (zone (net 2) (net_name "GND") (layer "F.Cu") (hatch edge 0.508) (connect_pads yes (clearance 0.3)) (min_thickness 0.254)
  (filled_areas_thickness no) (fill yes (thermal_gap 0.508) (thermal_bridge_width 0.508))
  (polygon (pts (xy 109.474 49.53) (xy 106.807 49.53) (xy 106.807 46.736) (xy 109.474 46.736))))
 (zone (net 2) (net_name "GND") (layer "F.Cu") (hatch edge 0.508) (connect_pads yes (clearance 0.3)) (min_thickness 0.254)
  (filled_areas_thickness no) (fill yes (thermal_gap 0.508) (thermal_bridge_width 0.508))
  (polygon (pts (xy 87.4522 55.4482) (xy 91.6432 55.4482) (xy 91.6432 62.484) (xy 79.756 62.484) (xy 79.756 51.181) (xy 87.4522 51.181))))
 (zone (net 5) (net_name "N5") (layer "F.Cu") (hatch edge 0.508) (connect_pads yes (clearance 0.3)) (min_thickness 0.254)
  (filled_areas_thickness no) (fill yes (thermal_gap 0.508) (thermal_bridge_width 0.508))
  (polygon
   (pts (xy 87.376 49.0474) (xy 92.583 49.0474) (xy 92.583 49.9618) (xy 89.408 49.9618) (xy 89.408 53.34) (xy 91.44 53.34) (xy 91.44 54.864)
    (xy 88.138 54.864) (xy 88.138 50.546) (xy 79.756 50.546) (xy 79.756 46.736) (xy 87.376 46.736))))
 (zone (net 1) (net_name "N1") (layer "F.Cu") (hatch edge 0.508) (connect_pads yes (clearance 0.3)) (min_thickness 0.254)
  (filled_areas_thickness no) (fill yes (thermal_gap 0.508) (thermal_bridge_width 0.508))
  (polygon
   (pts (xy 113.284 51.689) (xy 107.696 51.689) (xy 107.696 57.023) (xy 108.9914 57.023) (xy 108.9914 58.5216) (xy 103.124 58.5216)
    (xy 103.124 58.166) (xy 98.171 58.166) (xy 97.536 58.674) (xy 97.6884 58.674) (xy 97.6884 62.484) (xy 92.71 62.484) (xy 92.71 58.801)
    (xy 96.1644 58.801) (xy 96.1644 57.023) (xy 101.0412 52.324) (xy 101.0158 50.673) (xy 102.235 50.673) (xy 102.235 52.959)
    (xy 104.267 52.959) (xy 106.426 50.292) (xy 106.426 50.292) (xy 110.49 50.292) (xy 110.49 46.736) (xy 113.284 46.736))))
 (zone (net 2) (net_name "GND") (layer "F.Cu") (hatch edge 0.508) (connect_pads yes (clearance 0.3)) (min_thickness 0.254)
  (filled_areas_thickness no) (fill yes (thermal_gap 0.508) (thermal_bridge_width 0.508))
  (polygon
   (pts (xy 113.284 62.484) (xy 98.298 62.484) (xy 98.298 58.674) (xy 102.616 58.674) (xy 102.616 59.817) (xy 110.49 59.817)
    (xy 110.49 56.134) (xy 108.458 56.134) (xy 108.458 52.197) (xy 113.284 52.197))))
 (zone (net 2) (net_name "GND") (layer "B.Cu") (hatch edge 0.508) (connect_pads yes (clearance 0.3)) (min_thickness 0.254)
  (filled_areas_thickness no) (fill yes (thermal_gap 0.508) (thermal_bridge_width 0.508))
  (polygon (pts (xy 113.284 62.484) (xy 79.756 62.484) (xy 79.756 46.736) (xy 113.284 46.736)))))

